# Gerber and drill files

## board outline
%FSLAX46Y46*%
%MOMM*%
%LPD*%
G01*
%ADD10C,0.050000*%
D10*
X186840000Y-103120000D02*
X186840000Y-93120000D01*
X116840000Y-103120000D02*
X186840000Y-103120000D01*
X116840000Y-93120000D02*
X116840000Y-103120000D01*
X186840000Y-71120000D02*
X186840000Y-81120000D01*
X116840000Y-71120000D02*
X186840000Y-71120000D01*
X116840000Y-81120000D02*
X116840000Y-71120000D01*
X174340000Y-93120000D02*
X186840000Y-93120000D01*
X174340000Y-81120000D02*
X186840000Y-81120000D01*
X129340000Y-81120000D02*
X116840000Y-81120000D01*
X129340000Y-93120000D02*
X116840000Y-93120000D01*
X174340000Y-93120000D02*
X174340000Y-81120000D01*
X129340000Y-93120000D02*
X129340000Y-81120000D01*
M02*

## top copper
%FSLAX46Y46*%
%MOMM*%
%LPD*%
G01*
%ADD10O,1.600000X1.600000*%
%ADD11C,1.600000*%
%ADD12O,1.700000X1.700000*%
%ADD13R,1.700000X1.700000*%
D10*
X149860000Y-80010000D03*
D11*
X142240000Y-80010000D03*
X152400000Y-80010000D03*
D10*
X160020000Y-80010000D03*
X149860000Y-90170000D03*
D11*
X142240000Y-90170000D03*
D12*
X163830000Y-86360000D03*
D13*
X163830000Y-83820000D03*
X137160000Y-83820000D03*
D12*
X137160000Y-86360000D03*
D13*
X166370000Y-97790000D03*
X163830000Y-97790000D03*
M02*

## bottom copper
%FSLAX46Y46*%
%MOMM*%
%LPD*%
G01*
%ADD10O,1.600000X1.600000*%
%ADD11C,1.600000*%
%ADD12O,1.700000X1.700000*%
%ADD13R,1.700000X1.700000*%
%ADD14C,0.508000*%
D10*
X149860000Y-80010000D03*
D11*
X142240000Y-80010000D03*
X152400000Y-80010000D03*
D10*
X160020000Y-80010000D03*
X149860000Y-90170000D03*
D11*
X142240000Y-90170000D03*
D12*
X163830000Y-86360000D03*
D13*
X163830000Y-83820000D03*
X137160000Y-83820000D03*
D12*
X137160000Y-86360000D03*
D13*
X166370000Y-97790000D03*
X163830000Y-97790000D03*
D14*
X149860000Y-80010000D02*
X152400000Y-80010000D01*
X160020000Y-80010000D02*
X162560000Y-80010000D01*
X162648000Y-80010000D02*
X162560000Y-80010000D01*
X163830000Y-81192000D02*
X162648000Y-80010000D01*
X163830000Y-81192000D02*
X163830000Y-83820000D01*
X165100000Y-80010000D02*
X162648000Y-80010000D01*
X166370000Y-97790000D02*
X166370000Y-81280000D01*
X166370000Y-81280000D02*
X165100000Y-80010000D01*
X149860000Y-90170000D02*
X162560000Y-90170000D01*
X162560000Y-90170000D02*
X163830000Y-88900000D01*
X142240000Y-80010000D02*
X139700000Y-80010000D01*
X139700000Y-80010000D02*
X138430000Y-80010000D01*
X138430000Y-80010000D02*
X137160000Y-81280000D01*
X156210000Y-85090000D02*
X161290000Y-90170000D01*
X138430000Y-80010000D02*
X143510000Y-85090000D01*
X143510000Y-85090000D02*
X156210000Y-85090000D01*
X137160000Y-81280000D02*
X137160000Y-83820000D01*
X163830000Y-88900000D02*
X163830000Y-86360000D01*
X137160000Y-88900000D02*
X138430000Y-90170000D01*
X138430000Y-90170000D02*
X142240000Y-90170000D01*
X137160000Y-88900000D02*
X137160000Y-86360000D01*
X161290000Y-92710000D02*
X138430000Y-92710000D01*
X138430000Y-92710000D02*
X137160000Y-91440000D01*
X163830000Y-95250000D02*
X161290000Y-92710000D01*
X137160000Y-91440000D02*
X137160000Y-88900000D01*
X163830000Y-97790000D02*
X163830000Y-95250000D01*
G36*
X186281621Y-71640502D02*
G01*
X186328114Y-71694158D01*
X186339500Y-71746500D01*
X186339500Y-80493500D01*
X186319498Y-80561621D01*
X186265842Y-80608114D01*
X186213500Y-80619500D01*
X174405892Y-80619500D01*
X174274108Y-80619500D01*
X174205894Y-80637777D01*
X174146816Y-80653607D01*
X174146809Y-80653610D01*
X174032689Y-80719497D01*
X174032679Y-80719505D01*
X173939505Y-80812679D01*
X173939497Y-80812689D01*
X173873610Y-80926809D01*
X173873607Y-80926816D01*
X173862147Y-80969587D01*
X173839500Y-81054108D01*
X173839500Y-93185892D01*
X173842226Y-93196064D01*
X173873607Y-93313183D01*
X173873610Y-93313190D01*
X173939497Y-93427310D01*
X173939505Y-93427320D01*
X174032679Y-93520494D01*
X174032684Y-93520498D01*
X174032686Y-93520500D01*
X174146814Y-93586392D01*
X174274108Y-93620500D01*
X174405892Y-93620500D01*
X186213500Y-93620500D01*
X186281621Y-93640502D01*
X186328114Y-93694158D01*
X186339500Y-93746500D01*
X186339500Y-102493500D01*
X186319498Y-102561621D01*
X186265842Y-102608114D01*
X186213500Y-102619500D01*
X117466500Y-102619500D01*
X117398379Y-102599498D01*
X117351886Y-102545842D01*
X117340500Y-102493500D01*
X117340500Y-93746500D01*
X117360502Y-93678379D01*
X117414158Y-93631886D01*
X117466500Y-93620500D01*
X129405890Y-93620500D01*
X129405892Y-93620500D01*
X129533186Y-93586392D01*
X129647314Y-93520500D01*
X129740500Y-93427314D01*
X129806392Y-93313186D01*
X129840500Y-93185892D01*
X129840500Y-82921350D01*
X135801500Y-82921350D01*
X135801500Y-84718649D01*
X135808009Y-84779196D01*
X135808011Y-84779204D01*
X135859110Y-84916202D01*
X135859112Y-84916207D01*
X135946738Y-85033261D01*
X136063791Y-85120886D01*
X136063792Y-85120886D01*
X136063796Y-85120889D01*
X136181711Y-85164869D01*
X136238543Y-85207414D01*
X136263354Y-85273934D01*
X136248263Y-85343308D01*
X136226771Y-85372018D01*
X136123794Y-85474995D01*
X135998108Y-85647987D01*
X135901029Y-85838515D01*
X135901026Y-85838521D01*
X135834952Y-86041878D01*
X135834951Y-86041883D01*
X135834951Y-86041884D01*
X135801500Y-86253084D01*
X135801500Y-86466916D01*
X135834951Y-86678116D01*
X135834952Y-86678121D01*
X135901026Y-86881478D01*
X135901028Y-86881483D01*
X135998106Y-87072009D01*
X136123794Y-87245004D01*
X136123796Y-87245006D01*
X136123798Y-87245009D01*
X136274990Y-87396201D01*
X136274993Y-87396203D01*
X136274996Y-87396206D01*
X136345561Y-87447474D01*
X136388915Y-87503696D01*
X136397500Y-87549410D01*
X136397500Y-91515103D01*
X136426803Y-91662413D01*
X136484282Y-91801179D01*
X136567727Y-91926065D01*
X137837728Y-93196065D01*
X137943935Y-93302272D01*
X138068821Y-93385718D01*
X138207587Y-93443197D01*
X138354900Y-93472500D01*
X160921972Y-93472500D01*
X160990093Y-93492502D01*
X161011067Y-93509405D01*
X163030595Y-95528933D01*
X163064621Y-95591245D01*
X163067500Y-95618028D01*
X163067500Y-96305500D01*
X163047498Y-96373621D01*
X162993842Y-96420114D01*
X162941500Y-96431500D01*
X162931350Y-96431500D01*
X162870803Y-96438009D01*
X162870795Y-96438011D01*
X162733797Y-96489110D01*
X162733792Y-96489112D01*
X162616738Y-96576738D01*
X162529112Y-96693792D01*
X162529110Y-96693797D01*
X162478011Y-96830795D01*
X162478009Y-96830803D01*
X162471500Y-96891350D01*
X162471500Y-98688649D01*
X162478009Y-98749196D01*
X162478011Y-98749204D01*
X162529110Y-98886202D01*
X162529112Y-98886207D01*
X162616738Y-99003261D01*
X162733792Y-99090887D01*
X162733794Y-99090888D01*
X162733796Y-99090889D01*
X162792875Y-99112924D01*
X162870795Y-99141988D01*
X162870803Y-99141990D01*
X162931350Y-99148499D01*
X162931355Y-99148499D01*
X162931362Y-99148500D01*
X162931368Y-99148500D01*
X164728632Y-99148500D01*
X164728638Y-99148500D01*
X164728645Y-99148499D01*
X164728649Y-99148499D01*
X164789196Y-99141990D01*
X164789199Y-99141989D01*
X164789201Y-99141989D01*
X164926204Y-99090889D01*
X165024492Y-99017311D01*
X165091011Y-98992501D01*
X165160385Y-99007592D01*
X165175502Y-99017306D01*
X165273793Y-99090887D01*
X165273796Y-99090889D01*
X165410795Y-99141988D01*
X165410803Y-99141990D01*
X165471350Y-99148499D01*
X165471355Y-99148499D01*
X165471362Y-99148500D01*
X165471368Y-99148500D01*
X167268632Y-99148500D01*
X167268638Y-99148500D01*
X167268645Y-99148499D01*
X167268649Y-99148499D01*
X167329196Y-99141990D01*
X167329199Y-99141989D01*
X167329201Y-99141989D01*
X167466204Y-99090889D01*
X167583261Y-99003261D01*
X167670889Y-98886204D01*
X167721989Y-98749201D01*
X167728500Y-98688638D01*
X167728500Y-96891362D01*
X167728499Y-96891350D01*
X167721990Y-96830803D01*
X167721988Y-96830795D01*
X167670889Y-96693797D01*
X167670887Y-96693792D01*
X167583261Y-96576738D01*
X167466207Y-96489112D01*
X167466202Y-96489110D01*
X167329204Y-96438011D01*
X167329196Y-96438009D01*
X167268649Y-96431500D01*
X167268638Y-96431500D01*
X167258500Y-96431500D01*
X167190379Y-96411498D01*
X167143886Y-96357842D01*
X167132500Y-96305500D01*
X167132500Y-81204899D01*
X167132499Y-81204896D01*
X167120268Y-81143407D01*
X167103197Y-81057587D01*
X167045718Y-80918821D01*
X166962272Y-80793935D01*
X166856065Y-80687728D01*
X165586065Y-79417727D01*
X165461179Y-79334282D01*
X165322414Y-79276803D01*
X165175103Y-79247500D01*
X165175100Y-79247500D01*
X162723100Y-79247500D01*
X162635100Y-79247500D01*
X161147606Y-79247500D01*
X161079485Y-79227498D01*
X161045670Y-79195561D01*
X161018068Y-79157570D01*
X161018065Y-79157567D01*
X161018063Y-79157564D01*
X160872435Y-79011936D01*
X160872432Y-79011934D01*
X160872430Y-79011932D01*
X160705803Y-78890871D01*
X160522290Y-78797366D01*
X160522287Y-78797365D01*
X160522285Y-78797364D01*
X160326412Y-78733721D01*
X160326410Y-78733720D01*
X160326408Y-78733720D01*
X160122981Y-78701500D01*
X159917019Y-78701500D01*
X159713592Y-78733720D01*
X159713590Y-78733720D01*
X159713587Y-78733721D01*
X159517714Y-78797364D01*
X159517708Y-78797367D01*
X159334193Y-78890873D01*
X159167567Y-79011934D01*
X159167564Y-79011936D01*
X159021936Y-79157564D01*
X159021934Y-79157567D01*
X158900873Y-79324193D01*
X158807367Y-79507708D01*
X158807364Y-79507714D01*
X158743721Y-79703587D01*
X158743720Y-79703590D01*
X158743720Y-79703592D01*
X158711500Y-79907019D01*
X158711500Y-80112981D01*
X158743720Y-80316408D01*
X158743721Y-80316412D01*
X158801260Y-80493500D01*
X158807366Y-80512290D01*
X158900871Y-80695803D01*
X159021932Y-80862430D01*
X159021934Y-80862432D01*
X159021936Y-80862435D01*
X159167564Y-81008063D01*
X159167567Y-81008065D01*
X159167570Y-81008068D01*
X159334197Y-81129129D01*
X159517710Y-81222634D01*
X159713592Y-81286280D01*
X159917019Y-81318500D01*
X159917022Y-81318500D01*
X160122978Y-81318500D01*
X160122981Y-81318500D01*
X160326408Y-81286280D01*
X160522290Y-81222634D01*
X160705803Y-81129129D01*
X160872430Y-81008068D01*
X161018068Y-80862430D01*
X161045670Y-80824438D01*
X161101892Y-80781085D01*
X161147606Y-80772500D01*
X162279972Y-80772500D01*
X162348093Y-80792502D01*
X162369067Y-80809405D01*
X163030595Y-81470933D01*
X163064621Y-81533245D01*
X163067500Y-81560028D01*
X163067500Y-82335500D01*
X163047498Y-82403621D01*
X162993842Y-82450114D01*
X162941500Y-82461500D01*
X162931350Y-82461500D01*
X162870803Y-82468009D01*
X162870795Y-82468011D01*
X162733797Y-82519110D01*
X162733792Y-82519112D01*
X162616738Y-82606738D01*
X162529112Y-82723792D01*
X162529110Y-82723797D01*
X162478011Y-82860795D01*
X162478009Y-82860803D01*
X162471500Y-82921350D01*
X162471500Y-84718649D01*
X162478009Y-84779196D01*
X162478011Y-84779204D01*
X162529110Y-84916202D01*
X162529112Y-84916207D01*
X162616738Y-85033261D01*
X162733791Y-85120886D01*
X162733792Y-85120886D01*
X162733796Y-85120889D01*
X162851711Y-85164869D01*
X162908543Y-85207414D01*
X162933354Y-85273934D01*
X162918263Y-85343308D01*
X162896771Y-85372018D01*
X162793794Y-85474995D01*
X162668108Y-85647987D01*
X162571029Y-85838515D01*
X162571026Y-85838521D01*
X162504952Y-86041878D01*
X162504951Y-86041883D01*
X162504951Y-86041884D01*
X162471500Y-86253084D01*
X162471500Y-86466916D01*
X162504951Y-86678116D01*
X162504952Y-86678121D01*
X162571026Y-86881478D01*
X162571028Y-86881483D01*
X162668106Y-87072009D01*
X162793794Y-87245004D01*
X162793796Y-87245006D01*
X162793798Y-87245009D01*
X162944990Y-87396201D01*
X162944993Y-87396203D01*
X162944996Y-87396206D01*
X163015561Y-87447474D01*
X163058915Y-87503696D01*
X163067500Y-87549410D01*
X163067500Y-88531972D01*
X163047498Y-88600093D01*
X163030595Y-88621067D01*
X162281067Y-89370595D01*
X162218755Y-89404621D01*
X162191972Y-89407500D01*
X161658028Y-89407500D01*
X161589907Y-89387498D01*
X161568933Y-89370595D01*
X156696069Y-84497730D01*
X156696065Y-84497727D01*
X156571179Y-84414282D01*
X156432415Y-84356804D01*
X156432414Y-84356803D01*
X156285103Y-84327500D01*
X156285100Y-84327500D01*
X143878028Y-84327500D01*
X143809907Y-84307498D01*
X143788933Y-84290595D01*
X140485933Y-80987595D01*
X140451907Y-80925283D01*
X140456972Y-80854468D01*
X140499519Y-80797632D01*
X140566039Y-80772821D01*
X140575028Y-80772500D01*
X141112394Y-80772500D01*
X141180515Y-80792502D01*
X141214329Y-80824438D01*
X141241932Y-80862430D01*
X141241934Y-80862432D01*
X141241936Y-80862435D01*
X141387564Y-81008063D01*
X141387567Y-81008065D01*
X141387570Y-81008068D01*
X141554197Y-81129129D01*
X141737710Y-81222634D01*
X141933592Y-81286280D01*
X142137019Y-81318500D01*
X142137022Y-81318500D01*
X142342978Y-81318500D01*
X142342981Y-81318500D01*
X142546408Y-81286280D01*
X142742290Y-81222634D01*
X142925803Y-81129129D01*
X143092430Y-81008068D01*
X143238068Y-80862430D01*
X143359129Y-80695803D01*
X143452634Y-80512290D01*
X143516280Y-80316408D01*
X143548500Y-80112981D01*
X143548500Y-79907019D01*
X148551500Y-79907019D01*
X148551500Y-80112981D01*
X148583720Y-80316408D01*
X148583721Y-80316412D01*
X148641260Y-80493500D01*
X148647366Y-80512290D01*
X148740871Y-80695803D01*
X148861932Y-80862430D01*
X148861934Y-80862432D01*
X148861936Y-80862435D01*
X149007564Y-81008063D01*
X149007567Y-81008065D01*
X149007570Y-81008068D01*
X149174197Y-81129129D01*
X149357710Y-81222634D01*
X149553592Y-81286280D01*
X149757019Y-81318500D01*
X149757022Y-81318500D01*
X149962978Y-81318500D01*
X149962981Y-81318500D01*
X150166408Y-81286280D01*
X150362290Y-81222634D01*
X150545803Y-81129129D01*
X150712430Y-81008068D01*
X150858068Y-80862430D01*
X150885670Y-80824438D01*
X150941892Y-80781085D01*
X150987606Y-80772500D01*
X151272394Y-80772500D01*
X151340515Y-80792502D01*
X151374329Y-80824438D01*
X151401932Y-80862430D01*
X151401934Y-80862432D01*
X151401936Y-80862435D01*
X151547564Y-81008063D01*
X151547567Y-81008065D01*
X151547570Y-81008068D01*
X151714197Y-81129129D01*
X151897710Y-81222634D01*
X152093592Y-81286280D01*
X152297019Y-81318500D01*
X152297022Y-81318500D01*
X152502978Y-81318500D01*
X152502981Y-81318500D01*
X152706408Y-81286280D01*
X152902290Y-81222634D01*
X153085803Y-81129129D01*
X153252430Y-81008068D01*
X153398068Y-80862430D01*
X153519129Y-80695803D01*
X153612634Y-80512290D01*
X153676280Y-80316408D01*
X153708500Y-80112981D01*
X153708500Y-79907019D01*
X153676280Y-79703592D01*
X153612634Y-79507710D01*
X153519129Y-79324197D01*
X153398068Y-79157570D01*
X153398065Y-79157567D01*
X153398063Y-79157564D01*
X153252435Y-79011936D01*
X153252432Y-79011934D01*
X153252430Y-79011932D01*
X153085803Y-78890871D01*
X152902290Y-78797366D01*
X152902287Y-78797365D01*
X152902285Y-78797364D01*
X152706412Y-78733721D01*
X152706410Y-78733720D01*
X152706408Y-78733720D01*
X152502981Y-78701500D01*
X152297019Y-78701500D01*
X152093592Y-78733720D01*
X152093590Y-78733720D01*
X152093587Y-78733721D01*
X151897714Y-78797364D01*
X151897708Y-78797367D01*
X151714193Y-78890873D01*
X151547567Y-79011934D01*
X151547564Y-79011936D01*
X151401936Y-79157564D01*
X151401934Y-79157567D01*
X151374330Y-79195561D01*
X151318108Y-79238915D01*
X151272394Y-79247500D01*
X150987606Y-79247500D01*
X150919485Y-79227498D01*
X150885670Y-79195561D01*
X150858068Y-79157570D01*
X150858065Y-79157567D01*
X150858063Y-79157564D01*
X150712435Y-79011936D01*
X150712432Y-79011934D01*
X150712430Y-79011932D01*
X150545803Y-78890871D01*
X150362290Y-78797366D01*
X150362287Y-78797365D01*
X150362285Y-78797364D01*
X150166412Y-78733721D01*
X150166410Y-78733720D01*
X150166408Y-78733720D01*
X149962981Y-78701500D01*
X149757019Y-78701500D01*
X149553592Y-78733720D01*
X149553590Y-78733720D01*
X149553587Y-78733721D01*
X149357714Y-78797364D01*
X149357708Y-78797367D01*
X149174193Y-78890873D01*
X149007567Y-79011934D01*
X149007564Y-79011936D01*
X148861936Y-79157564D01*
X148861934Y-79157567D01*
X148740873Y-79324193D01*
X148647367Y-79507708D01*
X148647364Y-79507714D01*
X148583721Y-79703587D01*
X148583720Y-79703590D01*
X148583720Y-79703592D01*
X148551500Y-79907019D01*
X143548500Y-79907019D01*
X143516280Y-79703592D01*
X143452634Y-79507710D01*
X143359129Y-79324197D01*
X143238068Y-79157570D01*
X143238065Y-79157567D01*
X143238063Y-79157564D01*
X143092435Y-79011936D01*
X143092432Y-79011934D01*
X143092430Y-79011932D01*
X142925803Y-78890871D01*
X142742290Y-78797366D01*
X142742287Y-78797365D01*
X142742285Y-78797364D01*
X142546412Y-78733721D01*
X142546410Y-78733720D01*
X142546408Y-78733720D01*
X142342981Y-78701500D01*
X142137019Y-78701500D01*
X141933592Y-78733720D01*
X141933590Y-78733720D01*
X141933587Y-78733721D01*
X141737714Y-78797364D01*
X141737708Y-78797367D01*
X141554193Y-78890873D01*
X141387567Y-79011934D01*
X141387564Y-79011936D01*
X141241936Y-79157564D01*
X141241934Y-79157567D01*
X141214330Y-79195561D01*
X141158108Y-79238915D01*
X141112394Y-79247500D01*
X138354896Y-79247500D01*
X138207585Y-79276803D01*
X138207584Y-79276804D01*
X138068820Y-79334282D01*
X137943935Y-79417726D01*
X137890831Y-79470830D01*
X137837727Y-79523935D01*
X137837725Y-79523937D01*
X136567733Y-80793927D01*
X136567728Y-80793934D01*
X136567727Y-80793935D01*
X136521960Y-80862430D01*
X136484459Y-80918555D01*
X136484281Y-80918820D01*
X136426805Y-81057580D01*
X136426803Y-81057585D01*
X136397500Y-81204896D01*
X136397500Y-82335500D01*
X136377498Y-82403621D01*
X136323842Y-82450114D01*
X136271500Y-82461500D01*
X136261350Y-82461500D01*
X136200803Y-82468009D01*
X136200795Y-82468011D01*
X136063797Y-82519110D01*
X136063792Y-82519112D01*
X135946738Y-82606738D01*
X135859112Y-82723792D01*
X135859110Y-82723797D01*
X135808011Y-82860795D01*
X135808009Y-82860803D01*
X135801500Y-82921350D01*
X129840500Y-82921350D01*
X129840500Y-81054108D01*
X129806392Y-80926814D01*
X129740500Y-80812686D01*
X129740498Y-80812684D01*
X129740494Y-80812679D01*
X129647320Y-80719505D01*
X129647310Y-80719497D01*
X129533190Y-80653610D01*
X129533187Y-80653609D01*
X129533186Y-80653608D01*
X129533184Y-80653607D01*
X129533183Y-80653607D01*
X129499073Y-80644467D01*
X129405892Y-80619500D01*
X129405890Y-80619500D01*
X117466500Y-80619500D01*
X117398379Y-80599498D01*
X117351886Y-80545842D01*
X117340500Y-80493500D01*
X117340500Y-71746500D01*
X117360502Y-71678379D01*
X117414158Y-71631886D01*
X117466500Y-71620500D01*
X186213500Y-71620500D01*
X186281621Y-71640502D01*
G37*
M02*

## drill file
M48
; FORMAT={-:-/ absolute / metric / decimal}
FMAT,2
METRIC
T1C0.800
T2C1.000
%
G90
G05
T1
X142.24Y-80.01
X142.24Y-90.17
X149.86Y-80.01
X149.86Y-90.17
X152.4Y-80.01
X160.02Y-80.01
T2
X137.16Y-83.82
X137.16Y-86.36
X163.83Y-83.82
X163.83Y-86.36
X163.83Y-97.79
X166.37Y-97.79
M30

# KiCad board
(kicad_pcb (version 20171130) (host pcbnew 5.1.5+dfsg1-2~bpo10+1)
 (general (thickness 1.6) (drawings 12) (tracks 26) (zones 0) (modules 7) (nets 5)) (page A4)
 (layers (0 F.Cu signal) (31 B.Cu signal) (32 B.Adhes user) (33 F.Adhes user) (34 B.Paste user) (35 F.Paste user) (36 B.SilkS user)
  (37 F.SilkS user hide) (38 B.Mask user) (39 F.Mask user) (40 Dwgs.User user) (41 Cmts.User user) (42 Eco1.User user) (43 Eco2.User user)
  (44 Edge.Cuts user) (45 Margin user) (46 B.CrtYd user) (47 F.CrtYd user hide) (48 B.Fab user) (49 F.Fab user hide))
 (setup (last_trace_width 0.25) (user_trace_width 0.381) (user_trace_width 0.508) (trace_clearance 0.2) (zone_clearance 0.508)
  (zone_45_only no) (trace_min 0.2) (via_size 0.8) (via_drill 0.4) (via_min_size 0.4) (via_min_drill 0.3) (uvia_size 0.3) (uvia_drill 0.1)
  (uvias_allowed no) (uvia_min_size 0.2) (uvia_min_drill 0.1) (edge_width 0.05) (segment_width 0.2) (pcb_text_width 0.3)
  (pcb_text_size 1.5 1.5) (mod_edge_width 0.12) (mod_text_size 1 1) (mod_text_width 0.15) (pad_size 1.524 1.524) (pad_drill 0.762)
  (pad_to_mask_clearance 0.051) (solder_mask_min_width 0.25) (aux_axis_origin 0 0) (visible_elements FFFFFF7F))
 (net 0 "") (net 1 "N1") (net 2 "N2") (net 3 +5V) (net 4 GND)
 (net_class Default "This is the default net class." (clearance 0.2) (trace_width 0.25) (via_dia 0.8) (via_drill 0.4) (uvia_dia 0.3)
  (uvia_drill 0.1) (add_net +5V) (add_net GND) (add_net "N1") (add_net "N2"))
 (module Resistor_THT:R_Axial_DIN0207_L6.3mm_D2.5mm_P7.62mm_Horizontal (layer F.Cu) (at 142.24 80.01)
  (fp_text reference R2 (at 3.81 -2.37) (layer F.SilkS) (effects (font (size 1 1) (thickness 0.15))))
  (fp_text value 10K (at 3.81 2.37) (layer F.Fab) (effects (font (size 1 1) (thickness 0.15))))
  (pad 2 thru_hole oval (at 7.62 0) (size 1.6 1.6) (drill 0.8) (layers *.Cu *.Mask) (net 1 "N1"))
  (pad 1 thru_hole circle (at 0 0) (size 1.6 1.6) (drill 0.8) (layers *.Cu *.Mask) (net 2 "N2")))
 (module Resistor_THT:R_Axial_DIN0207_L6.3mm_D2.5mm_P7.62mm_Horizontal (layer F.Cu) (at 152.4 80.01)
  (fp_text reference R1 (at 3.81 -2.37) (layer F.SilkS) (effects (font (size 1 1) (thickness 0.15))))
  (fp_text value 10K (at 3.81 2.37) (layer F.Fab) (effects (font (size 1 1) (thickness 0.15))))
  (pad 1 thru_hole circle (at 0 0) (size 1.6 1.6) (drill 0.8) (layers *.Cu *.Mask) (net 1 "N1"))
  (pad 2 thru_hole oval (at 7.62 0) (size 1.6 1.6) (drill 0.8) (layers *.Cu *.Mask) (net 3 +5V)))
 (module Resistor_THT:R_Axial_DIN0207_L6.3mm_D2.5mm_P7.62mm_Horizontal (layer F.Cu) (at 142.24 90.17)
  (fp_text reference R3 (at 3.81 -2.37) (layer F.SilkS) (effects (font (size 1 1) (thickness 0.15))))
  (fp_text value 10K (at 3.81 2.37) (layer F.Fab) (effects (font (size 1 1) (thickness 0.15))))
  (pad 2 thru_hole oval (at 7.62 0) (size 1.6 1.6) (drill 0.8) (layers *.Cu *.Mask) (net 2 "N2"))
  (pad 1 thru_hole circle (at 0 0) (size 1.6 1.6) (drill 0.8) (layers *.Cu *.Mask) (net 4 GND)))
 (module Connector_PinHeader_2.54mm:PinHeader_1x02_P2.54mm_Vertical (layer F.Cu) (at 163.83 83.82)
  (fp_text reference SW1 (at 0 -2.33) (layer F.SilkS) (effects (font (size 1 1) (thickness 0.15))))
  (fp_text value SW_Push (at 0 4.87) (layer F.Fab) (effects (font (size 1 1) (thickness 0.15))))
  (pad 2 thru_hole oval (at 0 2.54) (size 1.7 1.7) (drill 1) (layers *.Cu *.Mask) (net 2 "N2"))
  (pad 1 thru_hole rect (at 0 0) (size 1.7 1.7) (drill 1) (layers *.Cu *.Mask) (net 3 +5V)))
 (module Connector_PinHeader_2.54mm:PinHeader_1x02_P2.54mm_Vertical (layer F.Cu) (at 137.16 83.82)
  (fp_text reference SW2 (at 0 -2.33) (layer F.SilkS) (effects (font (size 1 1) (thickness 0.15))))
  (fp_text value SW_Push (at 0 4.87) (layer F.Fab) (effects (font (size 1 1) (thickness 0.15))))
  (pad 1 thru_hole rect (at 0 0) (size 1.7 1.7) (drill 1) (layers *.Cu *.Mask) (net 2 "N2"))
  (pad 2 thru_hole oval (at 0 2.54) (size 1.7 1.7) (drill 1) (layers *.Cu *.Mask) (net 4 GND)))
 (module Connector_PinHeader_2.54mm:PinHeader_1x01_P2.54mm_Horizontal (layer F.Cu) (at 166.37 97.79 90)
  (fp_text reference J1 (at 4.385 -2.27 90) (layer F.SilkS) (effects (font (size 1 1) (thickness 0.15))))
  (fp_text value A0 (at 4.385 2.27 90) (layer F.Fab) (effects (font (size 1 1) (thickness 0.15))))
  (pad 1 thru_hole rect (at 0 0 90) (size 1.7 1.7) (drill 1) (layers *.Cu *.Mask) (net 3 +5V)))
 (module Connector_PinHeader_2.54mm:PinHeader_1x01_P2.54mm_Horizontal (layer F.Cu) (at 163.83 97.79 90)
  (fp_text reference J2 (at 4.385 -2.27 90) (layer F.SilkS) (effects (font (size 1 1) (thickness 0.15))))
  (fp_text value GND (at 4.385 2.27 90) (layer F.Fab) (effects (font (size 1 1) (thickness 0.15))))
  (pad 1 thru_hole rect (at 0 0 90) (size 1.7 1.7) (drill 1) (layers *.Cu *.Mask) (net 4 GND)))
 (gr_line (start 186.84 103.12) (end 186.84 93.12) (layer Edge.Cuts) (width 0.05))
 (gr_line (start 116.84 103.12) (end 186.84 103.12) (layer Edge.Cuts) (width 0.05))
 (gr_line (start 116.84 93.12) (end 116.84 103.12) (layer Edge.Cuts) (width 0.05))
 (gr_line (start 186.84 71.12) (end 186.84 81.12) (layer Edge.Cuts) (width 0.05))
 (gr_line (start 116.84 71.12) (end 186.84 71.12) (layer Edge.Cuts) (width 0.05))
 (gr_line (start 116.84 81.12) (end 116.84 71.12) (layer Edge.Cuts) (width 0.05))
 (gr_line (start 174.34 93.12) (end 186.84 93.12) (layer Edge.Cuts) (width 0.05))
 (gr_line (start 174.34 81.12) (end 186.84 81.12) (layer Edge.Cuts) (width 0.05))
 (gr_line (start 129.34 81.12) (end 116.84 81.12) (layer Edge.Cuts) (width 0.05))
 (gr_line (start 129.34 93.12) (end 116.84 93.12) (layer Edge.Cuts) (width 0.05))
 (gr_line (start 174.34 93.12) (end 174.34 81.12) (layer Edge.Cuts) (width 0.05))
 (gr_line (start 129.34 93.12) (end 129.34 81.12) (layer Edge.Cuts) (width 0.05))
 (segment (start 149.86 80.01) (end 152.4 80.01) (width 0.508) (layer B.Cu) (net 1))
 (segment (start 160.02 80.01) (end 162.56 80.01) (width 0.508) (layer B.Cu) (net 3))
 (segment (start 162.648 80.01) (end 162.56 80.01) (width 0.508) (layer B.Cu) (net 3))
 (segment (start 163.83 81.192) (end 162.648 80.01) (width 0.508) (layer B.Cu) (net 3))
 (segment (start 163.83 81.192) (end 163.83 83.82) (width 0.508) (layer B.Cu) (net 3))
 (segment (start 165.1 80.01) (end 162.648 80.01) (width 0.508) (layer B.Cu) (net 3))
 (segment (start 166.37 97.79) (end 166.37 81.28) (width 0.508) (layer B.Cu) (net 3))
 (segment (start 166.37 81.28) (end 165.1 80.01) (width 0.508) (layer B.Cu) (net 3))
 (segment (start 149.86 90.17) (end 162.56 90.17) (width 0.508) (layer B.Cu) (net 2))
 (segment (start 162.56 90.17) (end 163.83 88.9) (width 0.508) (layer B.Cu) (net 2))
 (segment (start 142.24 80.01) (end 139.7 80.01) (width 0.508) (layer B.Cu) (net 2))
 (segment (start 139.7 80.01) (end 138.43 80.01) (width 0.508) (layer B.Cu) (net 2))
 (segment (start 138.43 80.01) (end 137.16 81.28) (width 0.508) (layer B.Cu) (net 2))
 (segment (start 156.21 85.09) (end 161.29 90.17) (width 0.508) (layer B.Cu) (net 2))
 (segment (start 138.43 80.01) (end 143.51 85.09) (width 0.508) (layer B.Cu) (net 2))
 (segment (start 143.51 85.09) (end 156.21 85.09) (width 0.508) (layer B.Cu) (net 2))
 (segment (start 137.16 81.28) (end 137.16 83.82) (width 0.508) (layer B.Cu) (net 2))
 (segment (start 163.83 88.9) (end 163.83 86.36) (width 0.508) (layer B.Cu) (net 2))
 (segment (start 137.16 88.9) (end 138.43 90.17) (width 0.508) (layer B.Cu) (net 4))
 (segment (start 138.43 90.17) (end 142.24 90.17) (width 0.508) (layer B.Cu) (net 4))
 (segment (start 137.16 88.9) (end 137.16 86.36) (width 0.508) (layer B.Cu) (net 4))
 (segment (start 161.29 92.71) (end 138.43 92.71) (width 0.508) (layer B.Cu) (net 4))
 (segment (start 138.43 92.71) (end 137.16 91.44) (width 0.508) (layer B.Cu) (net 4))
 (segment (start 163.83 95.25) (end 161.29 92.71) (width 0.508) (layer B.Cu) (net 4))
 (segment (start 137.16 91.44) (end 137.16 88.9) (width 0.508) (layer B.Cu) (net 4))
 (segment (start 163.83 97.79) (end 163.83 95.25) (width 0.508) (layer B.Cu) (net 4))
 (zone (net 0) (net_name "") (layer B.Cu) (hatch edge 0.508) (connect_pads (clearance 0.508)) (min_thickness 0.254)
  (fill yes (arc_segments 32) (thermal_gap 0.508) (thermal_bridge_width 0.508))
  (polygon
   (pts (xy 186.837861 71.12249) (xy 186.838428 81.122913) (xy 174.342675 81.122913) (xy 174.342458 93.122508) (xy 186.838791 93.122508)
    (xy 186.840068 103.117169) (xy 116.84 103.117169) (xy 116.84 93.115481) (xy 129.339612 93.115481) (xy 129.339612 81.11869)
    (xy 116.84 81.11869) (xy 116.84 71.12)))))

